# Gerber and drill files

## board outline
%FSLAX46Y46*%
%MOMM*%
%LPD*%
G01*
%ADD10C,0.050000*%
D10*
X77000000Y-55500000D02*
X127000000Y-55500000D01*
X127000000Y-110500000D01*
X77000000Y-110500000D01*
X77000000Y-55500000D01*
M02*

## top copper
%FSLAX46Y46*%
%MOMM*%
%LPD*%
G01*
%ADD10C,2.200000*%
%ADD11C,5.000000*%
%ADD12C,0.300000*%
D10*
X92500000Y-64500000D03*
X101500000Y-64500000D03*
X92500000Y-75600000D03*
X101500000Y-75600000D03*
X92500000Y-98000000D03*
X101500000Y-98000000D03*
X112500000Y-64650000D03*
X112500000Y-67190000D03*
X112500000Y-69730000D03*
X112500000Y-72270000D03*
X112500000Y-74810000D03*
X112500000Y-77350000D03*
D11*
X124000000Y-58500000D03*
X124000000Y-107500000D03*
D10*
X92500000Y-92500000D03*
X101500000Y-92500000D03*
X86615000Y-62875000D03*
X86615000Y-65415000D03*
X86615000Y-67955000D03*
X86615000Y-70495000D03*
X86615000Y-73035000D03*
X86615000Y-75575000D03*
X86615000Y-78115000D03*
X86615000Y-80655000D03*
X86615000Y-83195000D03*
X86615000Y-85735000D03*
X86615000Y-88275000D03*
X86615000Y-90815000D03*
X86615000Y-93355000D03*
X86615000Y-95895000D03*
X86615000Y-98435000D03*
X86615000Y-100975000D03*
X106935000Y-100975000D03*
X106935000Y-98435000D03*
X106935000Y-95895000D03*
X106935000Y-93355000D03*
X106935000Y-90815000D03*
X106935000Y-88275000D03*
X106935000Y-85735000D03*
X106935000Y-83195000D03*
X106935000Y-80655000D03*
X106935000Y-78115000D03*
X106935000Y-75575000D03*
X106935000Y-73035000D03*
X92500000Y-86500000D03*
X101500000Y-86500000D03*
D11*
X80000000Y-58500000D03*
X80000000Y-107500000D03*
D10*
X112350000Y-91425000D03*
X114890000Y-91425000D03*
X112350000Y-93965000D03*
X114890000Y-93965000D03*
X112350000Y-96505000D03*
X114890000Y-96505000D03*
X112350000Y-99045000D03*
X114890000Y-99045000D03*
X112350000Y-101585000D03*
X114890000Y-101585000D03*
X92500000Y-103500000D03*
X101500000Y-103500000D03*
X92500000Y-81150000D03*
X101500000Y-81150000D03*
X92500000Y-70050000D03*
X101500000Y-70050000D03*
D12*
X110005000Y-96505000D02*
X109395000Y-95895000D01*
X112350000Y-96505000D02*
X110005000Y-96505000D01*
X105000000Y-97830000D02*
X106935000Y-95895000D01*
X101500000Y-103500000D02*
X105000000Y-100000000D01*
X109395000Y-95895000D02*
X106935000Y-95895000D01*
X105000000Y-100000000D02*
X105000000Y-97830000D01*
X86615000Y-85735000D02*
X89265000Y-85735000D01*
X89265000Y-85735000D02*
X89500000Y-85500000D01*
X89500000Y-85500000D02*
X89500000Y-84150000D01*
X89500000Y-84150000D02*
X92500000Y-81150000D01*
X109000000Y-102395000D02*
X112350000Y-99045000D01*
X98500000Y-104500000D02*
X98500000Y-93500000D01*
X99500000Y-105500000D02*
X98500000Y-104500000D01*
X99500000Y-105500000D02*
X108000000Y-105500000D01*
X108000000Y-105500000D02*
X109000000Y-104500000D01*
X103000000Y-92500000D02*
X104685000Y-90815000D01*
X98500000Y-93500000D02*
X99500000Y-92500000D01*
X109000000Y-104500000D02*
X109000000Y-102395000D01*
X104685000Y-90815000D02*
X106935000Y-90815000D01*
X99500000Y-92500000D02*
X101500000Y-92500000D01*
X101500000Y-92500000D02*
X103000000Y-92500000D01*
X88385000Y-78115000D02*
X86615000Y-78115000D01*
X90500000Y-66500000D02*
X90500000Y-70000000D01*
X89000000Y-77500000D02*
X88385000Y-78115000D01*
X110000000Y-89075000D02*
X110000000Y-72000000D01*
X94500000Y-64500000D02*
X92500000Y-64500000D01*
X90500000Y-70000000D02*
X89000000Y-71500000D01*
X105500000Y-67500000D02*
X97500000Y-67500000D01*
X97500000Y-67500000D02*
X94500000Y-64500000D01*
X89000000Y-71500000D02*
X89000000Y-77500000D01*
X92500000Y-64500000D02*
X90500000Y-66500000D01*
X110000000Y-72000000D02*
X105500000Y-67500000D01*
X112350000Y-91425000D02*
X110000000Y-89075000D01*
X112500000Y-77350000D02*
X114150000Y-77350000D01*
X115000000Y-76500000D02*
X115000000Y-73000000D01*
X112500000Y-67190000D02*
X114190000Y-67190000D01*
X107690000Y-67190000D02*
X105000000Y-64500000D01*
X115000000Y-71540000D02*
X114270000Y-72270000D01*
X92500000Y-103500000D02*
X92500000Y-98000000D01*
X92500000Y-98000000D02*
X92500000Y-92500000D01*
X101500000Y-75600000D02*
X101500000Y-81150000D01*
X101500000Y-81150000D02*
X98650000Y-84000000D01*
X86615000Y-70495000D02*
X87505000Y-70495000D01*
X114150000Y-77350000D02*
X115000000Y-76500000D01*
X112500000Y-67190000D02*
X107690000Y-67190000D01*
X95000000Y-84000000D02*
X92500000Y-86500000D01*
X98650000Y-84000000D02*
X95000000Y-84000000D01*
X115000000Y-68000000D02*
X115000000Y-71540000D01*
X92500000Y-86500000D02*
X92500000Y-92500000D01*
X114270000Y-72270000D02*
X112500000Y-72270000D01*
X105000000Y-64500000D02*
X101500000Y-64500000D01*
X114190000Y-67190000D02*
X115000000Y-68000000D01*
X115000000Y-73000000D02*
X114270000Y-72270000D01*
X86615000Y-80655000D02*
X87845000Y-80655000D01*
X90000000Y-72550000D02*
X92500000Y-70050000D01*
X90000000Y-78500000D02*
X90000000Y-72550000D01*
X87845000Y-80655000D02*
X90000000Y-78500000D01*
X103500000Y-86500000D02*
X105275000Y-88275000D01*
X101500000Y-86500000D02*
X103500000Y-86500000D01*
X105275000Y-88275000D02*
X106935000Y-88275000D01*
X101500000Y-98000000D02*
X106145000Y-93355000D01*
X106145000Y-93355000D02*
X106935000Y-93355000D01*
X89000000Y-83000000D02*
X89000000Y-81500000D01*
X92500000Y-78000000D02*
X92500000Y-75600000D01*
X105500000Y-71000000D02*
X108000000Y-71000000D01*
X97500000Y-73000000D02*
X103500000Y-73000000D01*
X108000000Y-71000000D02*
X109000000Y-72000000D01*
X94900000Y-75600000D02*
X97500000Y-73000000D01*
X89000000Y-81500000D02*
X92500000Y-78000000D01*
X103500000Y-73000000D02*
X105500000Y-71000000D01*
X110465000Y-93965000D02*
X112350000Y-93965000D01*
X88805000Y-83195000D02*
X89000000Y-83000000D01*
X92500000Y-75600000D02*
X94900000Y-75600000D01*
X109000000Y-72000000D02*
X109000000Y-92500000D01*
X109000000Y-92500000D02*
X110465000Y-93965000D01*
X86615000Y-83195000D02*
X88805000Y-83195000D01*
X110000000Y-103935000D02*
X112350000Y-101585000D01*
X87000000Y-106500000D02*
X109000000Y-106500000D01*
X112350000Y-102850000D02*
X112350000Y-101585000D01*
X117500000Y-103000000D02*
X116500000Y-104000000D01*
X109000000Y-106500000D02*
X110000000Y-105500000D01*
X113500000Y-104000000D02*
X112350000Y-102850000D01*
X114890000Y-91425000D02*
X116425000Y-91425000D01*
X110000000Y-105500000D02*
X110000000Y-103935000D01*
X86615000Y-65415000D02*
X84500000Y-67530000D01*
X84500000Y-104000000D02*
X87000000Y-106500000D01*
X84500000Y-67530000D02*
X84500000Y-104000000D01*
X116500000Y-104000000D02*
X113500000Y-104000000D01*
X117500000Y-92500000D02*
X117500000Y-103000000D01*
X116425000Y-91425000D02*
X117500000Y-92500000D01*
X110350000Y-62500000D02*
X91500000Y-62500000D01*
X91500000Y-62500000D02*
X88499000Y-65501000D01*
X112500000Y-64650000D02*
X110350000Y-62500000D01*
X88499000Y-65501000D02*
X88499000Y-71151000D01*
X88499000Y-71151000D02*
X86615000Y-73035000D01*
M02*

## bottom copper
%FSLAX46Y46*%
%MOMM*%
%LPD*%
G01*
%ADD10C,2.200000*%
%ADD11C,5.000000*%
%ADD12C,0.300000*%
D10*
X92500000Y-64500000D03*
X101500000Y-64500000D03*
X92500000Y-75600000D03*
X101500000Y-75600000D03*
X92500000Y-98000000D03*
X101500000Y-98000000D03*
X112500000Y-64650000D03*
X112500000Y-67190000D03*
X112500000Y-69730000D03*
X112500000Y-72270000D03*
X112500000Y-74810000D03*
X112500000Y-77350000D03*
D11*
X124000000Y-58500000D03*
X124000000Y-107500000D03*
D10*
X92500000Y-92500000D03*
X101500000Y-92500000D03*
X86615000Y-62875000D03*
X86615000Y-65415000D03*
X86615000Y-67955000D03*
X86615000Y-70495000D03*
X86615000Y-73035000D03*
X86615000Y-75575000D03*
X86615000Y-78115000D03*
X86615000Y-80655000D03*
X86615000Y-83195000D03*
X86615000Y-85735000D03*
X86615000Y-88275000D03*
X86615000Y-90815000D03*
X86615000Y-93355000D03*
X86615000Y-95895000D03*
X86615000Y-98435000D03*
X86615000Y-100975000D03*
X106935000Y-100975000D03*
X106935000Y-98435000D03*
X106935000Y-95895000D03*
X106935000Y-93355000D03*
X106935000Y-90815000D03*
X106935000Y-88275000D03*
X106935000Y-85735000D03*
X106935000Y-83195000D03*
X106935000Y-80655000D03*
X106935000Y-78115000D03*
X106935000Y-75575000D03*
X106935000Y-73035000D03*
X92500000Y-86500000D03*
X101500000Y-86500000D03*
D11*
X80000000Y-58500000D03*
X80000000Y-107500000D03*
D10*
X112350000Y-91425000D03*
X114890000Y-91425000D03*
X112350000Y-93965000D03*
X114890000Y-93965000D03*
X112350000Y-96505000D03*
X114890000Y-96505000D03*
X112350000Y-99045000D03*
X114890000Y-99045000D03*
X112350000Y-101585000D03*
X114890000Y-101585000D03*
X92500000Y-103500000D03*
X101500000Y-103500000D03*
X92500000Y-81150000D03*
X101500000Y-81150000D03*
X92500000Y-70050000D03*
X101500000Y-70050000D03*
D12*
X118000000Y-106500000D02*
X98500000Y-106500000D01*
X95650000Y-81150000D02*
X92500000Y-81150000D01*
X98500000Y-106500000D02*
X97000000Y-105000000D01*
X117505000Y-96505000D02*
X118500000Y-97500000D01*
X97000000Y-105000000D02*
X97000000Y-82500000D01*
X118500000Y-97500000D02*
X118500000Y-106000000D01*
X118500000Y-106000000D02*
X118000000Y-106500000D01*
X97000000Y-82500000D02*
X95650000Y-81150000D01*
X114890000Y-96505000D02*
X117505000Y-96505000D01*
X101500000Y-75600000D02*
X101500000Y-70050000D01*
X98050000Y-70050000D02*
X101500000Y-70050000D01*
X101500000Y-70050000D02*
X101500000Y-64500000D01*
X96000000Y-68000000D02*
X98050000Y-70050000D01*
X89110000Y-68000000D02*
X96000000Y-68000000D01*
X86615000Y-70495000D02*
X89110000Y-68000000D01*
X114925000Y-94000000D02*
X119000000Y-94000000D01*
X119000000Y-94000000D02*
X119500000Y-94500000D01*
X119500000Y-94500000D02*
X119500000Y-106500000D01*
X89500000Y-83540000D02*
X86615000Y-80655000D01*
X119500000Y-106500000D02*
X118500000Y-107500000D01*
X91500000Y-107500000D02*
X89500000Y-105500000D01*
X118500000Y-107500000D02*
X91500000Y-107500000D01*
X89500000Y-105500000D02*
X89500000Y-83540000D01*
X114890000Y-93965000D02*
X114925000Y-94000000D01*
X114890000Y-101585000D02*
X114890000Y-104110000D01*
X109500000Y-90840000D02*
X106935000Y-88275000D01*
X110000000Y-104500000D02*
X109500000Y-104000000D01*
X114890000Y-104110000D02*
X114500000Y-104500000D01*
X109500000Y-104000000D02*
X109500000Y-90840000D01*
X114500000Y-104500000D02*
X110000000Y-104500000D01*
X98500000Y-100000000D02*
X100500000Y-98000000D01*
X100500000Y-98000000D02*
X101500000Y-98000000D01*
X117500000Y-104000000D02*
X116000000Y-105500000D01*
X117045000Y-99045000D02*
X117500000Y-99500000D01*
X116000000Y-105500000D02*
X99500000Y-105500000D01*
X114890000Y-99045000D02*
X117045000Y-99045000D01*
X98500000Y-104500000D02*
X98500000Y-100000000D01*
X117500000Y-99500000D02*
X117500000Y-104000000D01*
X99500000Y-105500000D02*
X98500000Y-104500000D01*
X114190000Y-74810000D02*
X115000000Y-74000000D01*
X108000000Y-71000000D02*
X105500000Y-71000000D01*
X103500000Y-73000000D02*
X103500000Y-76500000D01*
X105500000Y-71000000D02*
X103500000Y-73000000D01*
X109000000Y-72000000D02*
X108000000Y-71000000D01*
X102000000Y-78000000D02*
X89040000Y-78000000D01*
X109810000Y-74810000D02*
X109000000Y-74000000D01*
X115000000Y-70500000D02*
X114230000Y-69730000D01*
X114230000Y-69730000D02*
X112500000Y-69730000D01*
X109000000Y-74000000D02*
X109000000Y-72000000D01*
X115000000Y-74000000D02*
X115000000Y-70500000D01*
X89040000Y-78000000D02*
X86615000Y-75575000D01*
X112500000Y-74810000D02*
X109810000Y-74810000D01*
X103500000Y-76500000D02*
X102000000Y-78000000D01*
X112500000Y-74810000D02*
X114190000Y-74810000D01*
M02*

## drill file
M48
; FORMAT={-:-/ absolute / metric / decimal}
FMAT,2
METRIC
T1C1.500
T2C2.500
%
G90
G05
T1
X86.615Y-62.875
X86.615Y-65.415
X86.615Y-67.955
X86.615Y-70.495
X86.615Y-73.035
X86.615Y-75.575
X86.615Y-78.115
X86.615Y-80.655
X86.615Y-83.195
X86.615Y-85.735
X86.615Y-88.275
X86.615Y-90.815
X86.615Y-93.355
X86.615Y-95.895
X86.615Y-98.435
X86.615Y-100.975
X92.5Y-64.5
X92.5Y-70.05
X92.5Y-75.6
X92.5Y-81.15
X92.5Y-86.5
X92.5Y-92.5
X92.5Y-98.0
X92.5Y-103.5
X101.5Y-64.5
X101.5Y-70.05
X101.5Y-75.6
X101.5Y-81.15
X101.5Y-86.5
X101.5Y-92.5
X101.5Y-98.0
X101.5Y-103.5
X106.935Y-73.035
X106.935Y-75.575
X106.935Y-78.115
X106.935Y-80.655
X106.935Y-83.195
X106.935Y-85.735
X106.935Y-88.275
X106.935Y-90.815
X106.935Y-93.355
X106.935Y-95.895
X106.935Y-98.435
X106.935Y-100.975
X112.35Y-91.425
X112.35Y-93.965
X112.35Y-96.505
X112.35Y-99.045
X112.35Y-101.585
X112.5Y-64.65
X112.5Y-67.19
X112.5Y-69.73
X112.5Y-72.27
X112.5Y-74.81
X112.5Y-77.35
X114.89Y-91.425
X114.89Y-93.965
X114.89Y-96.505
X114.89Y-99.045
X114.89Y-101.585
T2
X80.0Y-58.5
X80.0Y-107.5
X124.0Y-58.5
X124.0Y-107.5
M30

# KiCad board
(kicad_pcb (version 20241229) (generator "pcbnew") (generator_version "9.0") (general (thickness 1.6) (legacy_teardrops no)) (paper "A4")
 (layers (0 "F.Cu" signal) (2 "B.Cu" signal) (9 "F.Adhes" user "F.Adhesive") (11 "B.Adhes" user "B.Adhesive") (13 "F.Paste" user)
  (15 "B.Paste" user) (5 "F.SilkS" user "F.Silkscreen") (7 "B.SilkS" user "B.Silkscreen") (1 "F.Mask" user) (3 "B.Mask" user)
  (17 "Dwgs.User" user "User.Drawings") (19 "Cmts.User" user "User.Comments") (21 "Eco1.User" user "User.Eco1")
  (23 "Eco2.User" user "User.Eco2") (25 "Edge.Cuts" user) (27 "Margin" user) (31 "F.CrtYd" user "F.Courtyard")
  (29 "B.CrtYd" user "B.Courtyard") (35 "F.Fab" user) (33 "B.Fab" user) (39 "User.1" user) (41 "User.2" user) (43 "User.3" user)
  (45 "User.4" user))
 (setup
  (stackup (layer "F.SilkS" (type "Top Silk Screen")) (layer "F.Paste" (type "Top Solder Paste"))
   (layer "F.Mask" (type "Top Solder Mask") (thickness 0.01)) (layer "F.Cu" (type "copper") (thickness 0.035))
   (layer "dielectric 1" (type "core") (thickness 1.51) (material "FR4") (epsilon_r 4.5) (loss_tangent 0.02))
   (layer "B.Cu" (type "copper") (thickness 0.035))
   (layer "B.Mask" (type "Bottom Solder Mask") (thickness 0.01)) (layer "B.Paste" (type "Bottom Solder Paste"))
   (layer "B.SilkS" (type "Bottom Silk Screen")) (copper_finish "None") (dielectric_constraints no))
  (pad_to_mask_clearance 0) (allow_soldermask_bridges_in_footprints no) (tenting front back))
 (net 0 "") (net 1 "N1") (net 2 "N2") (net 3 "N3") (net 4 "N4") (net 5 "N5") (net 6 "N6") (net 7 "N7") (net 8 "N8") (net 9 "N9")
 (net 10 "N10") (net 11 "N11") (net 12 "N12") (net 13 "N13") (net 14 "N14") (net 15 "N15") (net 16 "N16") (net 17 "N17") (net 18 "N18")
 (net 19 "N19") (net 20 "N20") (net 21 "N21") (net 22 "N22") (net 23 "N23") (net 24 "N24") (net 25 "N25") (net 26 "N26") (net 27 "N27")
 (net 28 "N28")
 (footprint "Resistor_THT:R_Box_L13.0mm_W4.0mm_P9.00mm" (layer "F.Cu") (at 92.5 64.5)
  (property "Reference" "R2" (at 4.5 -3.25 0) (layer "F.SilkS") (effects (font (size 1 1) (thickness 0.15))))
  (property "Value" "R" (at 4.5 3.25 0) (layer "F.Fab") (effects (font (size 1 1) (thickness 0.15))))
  (pad "1" thru_hole circle (at 0 0) (size 2.2 2.2) (drill 1.5) (layers "*.Cu" "*.Mask") (remove_unused_layers no) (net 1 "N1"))
  (pad "2" thru_hole circle (at 9 0) (size 2.2 2.2) (drill 1.5) (layers "*.Cu" "*.Mask") (remove_unused_layers no) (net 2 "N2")))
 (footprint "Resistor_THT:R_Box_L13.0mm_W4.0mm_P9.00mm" (layer "F.Cu") (at 92.5 75.6)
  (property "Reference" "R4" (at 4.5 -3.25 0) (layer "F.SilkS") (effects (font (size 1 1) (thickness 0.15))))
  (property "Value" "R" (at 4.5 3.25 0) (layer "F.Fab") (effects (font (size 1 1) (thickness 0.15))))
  (pad "1" thru_hole circle (at 0 0) (size 2.2 2.2) (drill 1.5) (layers "*.Cu" "*.Mask") (remove_unused_layers no) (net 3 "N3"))
  (pad "2" thru_hole circle (at 9 0) (size 2.2 2.2) (drill 1.5) (layers "*.Cu" "*.Mask") (remove_unused_layers no) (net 2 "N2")))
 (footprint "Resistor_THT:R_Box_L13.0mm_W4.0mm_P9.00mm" (layer "F.Cu") (at 92.5 98)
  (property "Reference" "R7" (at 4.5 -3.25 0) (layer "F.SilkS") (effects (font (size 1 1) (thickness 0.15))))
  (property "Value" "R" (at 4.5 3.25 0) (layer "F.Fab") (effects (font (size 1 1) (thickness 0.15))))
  (pad "1" thru_hole circle (at 0 0) (size 2.2 2.2) (drill 1.5) (layers "*.Cu" "*.Mask") (remove_unused_layers no) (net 2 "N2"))
  (pad "2" thru_hole circle (at 9 0) (size 2.2 2.2) (drill 1.5) (layers "*.Cu" "*.Mask") (remove_unused_layers no) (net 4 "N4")))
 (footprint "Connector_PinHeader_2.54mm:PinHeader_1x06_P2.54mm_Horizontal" (layer "F.Cu") (at 112.5 64.65)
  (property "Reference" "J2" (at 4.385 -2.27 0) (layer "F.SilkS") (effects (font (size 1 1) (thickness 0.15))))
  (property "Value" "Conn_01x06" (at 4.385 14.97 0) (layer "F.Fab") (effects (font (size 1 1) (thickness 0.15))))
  (pad "1" thru_hole circle (at 0 0) (size 2.2 2.2) (drill 1.5) (layers "*.Cu" "*.Mask") (remove_unused_layers no) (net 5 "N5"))
  (pad "2" thru_hole circle (at 0 2.54) (size 2.2 2.2) (drill 1.5) (layers "*.Cu" "*.Mask") (remove_unused_layers no) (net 2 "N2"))
  (pad "3" thru_hole circle (at 0 5.08) (size 2.2 2.2) (drill 1.5) (layers "*.Cu" "*.Mask") (remove_unused_layers no) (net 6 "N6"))
  (pad "4" thru_hole circle (at 0 7.62) (size 2.2 2.2) (drill 1.5) (layers "*.Cu" "*.Mask") (remove_unused_layers no) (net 2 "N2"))
  (pad "5" thru_hole circle (at 0 10.16) (size 2.2 2.2) (drill 1.5) (layers "*.Cu" "*.Mask") (remove_unused_layers no) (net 6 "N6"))
  (pad "6" thru_hole circle (at 0 12.7) (size 2.2 2.2) (drill 1.5) (layers "*.Cu" "*.Mask") (remove_unused_layers no) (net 2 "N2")))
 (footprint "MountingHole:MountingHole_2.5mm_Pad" (layer "F.Cu") (at 124 58.5)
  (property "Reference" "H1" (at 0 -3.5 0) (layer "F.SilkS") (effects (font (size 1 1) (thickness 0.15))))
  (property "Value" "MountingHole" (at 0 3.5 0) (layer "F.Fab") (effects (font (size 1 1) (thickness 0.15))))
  (pad "1" thru_hole circle (at 0 0) (size 5 5) (drill 2.5) (layers "*.Cu" "*.Mask") (remove_unused_layers no)))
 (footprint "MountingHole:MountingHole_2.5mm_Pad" (layer "F.Cu") (at 124 107.5)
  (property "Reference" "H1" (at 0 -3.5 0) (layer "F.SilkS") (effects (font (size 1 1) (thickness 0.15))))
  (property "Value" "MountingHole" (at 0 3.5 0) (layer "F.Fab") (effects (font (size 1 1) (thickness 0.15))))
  (pad "1" thru_hole circle (at 0 0) (size 5 5) (drill 2.5) (layers "*.Cu" "*.Mask") (remove_unused_layers no)))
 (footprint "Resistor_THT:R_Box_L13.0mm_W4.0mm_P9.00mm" (layer "F.Cu") (at 92.5 92.5)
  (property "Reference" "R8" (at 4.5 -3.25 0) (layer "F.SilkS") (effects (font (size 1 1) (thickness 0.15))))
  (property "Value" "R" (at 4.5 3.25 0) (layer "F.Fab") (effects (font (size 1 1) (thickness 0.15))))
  (pad "1" thru_hole circle (at 0 0) (size 2.2 2.2) (drill 1.5) (layers "*.Cu" "*.Mask") (remove_unused_layers no) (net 2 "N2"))
  (pad "2" thru_hole circle (at 9 0) (size 2.2 2.2) (drill 1.5) (layers "*.Cu" "*.Mask") (remove_unused_layers no) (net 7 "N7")))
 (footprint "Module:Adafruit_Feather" (layer "F.Cu") (at 86.615 62.875)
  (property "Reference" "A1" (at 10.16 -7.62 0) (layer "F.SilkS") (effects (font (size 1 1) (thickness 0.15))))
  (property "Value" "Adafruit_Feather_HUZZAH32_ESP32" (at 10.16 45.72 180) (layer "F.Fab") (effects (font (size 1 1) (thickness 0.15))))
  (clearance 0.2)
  (pad "1" thru_hole circle (at 0 0) (size 2.2 2.2) (drill 1.5) (layers "*.Cu" "*.Mask") (remove_unused_layers no) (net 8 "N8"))
  (pad "2" thru_hole circle (at 0 2.54) (size 2.2 2.2) (drill 1.5) (layers "*.Cu" "*.Mask") (remove_unused_layers no) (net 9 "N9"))
  (pad "3" thru_hole circle (at 0 5.08) (size 2.2 2.2) (drill 1.5) (layers "*.Cu" "*.Mask") (remove_unused_layers no) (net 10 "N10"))
  (pad "4" thru_hole circle (at 0 7.62) (size 2.2 2.2) (drill 1.5) (layers "*.Cu" "*.Mask") (remove_unused_layers no) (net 2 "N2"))
  (pad "5" thru_hole circle (at 0 10.16) (size 2.2 2.2) (drill 1.5) (layers "*.Cu" "*.Mask") (remove_unused_layers no) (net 5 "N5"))
  (pad "6" thru_hole circle (at 0 12.7) (size 2.2 2.2) (drill 1.5) (layers "*.Cu" "*.Mask") (remove_unused_layers no) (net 6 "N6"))
  (pad "7" thru_hole circle (at 0 15.24) (size 2.2 2.2) (drill 1.5) (layers "*.Cu" "*.Mask") (remove_unused_layers no) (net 1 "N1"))
  (pad "8" thru_hole circle (at 0 17.78) (size 2.2 2.2) (drill 1.5) (layers "*.Cu" "*.Mask") (remove_unused_layers no) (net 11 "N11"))
  (pad "9" thru_hole circle (at 0 20.32) (size 2.2 2.2) (drill 1.5) (layers "*.Cu" "*.Mask") (remove_unused_layers no) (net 3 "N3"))
  (pad "10" thru_hole circle (at 0 22.86) (size 2.2 2.2) (drill 1.5) (layers "*.Cu" "*.Mask") (remove_unused_layers no) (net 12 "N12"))
  (pad "11" thru_hole circle (at 0 25.4) (size 2.2 2.2) (drill 1.5) (layers "*.Cu" "*.Mask") (remove_unused_layers no) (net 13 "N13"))
  (pad "12" thru_hole circle (at 0 27.94) (size 2.2 2.2) (drill 1.5) (layers "*.Cu" "*.Mask") (remove_unused_layers no) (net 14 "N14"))
  (pad "13" thru_hole circle (at 0 30.48) (size 2.2 2.2) (drill 1.5) (layers "*.Cu" "*.Mask") (remove_unused_layers no) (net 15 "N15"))
  (pad "14" thru_hole circle (at 0 33.02) (size 2.2 2.2) (drill 1.5) (layers "*.Cu" "*.Mask") (remove_unused_layers no) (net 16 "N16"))
  (pad "15" thru_hole circle (at 0 35.56) (size 2.2 2.2) (drill 1.5) (layers "*.Cu" "*.Mask") (remove_unused_layers no) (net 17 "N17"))
  (pad "16" thru_hole circle (at 0 38.1) (size 2.2 2.2) (drill 1.5) (layers "*.Cu" "*.Mask") (remove_unused_layers no) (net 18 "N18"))
  (pad "17" thru_hole circle (at 20.32 38.1) (size 2.2 2.2) (drill 1.5) (layers "*.Cu" "*.Mask") (remove_unused_layers no) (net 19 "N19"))
  (pad "18" thru_hole circle (at 20.32 35.56) (size 2.2 2.2) (drill 1.5) (layers "*.Cu" "*.Mask") (remove_unused_layers no) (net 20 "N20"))
  (pad "19" thru_hole circle (at 20.32 33.02) (size 2.2 2.2) (drill 1.5) (layers "*.Cu" "*.Mask") (remove_unused_layers no) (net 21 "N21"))
  (pad "20" thru_hole circle (at 20.32 30.48) (size 2.2 2.2) (drill 1.5) (layers "*.Cu" "*.Mask") (remove_unused_layers no) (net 4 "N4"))
  (pad "21" thru_hole circle (at 20.32 27.94) (size 2.2 2.2) (drill 1.5) (layers "*.Cu" "*.Mask") (remove_unused_layers no) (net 7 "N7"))
  (pad "22" thru_hole circle (at 20.32 25.4) (size 2.2 2.2) (drill 1.5) (layers "*.Cu" "*.Mask") (remove_unused_layers no) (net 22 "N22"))
  (pad "23" thru_hole circle (at 20.32 22.86) (size 2.2 2.2) (drill 1.5) (layers "*.Cu" "*.Mask") (remove_unused_layers no) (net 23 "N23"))
  (pad "24" thru_hole circle (at 20.32 20.32) (size 2.2 2.2) (drill 1.5) (layers "*.Cu" "*.Mask") (remove_unused_layers no) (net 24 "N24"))
  (pad "25" thru_hole circle (at 20.32 17.78) (size 2.2 2.2) (drill 1.5) (layers "*.Cu" "*.Mask") (remove_unused_layers no) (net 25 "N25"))
  (pad "26" thru_hole circle (at 20.32 15.24) (size 2.2 2.2) (drill 1.5) (layers "*.Cu" "*.Mask") (remove_unused_layers no) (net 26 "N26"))
  (pad "27" thru_hole circle (at 20.32 12.7) (size 2.2 2.2) (drill 1.5) (layers "*.Cu" "*.Mask") (remove_unused_layers no) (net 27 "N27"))
  (pad "28" thru_hole circle (at 20.32 10.16) (size 2.2 2.2) (drill 1.5) (layers "*.Cu" "*.Mask") (remove_unused_layers no) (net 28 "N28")))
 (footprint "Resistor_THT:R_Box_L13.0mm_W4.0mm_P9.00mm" (layer "F.Cu") (at 92.5 86.5)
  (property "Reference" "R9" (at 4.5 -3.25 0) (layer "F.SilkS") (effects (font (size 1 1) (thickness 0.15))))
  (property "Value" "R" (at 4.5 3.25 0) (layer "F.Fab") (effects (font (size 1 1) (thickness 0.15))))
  (pad "1" thru_hole circle (at 0 0) (size 2.2 2.2) (drill 1.5) (layers "*.Cu" "*.Mask") (remove_unused_layers no) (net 2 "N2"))
  (pad "2" thru_hole circle (at 9 0) (size 2.2 2.2) (drill 1.5) (layers "*.Cu" "*.Mask") (remove_unused_layers no) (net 22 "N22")))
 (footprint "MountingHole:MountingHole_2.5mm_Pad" (layer "F.Cu") (at 80 58.5)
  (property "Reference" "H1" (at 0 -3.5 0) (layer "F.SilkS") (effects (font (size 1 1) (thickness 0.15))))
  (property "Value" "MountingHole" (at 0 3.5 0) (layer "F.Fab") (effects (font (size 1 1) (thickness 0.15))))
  (pad "1" thru_hole circle (at 0 0) (size 5 5) (drill 2.5) (layers "*.Cu" "*.Mask") (remove_unused_layers no)))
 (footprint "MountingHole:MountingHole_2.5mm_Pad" (layer "F.Cu") (at 80 107.5)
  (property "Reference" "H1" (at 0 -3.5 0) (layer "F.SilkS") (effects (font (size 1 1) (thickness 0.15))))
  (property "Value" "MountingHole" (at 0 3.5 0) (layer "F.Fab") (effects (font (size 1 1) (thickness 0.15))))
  (pad "1" thru_hole circle (at 0 0) (size 5 5) (drill 2.5) (layers "*.Cu" "*.Mask") (remove_unused_layers no)))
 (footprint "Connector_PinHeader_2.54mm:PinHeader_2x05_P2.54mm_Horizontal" (layer "F.Cu") (at 112.35 91.425)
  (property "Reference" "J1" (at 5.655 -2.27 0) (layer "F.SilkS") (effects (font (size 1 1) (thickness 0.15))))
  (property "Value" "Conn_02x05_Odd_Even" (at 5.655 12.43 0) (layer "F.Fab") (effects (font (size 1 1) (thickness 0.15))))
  (pad "1" thru_hole circle (at 0 0) (size 2.2 2.2) (drill 1.5) (layers "*.Cu" "*.Mask") (remove_unused_layers no) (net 1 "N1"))
  (pad "2" thru_hole circle (at 2.54 0) (size 2.2 2.2) (drill 1.5) (layers "*.Cu" "*.Mask") (remove_unused_layers no) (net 9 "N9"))
  (pad "3" thru_hole circle (at 0 2.54) (size 2.2 2.2) (drill 1.5) (layers "*.Cu" "*.Mask") (remove_unused_layers no) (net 3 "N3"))
  (pad "4" thru_hole circle (at 2.54 2.54) (size 2.2 2.2) (drill 1.5) (layers "*.Cu" "*.Mask") (remove_unused_layers no) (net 11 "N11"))
  (pad "5" thru_hole circle (at 0 5.08) (size 2.2 2.2) (drill 1.5) (layers "*.Cu" "*.Mask") (remove_unused_layers no) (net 21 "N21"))
  (pad "6" thru_hole circle (at 2.54 5.08) (size 2.2 2.2) (drill 1.5) (layers "*.Cu" "*.Mask") (remove_unused_layers no) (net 12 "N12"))
  (pad "7" thru_hole circle (at 0 7.62) (size 2.2 2.2) (drill 1.5) (layers "*.Cu" "*.Mask") (remove_unused_layers no) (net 7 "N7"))
  (pad "8" thru_hole circle (at 2.54 7.62) (size 2.2 2.2) (drill 1.5) (layers "*.Cu" "*.Mask") (remove_unused_layers no) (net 4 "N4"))
  (pad "9" thru_hole circle (at 0 10.16) (size 2.2 2.2) (drill 1.5) (layers "*.Cu" "*.Mask") (remove_unused_layers no) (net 9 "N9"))
  (pad "10" thru_hole circle (at 2.54 10.16) (size 2.2 2.2) (drill 1.5) (layers "*.Cu" "*.Mask") (remove_unused_layers no) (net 22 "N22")))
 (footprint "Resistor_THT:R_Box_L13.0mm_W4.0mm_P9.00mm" (layer "F.Cu") (at 92.5 103.5)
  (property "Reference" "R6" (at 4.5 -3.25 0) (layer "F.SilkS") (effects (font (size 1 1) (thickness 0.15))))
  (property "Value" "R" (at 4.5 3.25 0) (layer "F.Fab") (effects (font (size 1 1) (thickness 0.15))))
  (pad "1" thru_hole circle (at 0 0) (size 2.2 2.2) (drill 1.5) (layers "*.Cu" "*.Mask") (remove_unused_layers no) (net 2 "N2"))
  (pad "2" thru_hole circle (at 9 0) (size 2.2 2.2) (drill 1.5) (layers "*.Cu" "*.Mask") (remove_unused_layers no) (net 21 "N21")))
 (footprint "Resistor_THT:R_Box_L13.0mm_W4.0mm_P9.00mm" (layer "F.Cu") (at 92.5 81.15)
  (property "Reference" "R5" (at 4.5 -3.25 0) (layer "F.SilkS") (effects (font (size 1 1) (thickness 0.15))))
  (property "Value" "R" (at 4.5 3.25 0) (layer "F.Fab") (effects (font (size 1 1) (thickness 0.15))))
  (pad "1" thru_hole circle (at 0 0) (size 2.2 2.2) (drill 1.5) (layers "*.Cu" "*.Mask") (remove_unused_layers no) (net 12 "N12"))
  (pad "2" thru_hole circle (at 9 0) (size 2.2 2.2) (drill 1.5) (layers "*.Cu" "*.Mask") (remove_unused_layers no) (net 2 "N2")))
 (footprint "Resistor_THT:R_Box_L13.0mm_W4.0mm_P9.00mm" (layer "F.Cu") (at 92.5 70.05)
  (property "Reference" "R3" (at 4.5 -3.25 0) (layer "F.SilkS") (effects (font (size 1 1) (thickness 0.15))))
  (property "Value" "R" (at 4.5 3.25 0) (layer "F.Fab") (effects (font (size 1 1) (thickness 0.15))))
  (pad "1" thru_hole circle (at 0 0) (size 2.2 2.2) (drill 1.5) (layers "*.Cu" "*.Mask") (remove_unused_layers no) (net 11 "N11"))
  (pad "2" thru_hole circle (at 9 0) (size 2.2 2.2) (drill 1.5) (layers "*.Cu" "*.Mask") (remove_unused_layers no) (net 2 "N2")))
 (gr_rect (start 77 55.5) (end 127 110.5) (stroke (width 0.05) (type default)) (fill no) (layer "Edge.Cuts"))
 (segment (start 110.005 96.505) (end 109.395 95.895) (width 0.3) (layer "F.Cu") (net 21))
 (segment (start 112.35 96.505) (end 110.005 96.505) (width 0.3) (layer "F.Cu") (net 21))
 (segment (start 105 97.83) (end 106.935 95.895) (width 0.3) (layer "F.Cu") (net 21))
 (segment (start 101.5 103.5) (end 105 100) (width 0.3) (layer "F.Cu") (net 21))
 (segment (start 109.395 95.895) (end 106.935 95.895) (width 0.3) (layer "F.Cu") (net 21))
 (segment (start 105 100) (end 105 97.83) (width 0.3) (layer "F.Cu") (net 21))
 (segment (start 86.615 85.735) (end 89.265 85.735) (width 0.3) (layer "F.Cu") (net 12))
 (segment (start 89.265 85.735) (end 89.5 85.5) (width 0.3) (layer "F.Cu") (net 12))
 (segment (start 89.5 85.5) (end 89.5 84.15) (width 0.3) (layer "F.Cu") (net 12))
 (segment (start 89.5 84.15) (end 92.5 81.15) (width 0.3) (layer "F.Cu") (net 12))
 (segment (start 118 106.5) (end 98.5 106.5) (width 0.3) (layer "B.Cu") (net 12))
 (segment (start 95.65 81.15) (end 92.5 81.15) (width 0.3) (layer "B.Cu") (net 12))
 (segment (start 98.5 106.5) (end 97 105) (width 0.3) (layer "B.Cu") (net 12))
 (segment (start 117.505 96.505) (end 118.5 97.5) (width 0.3) (layer "B.Cu") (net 12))
 (segment (start 97 105) (end 97 82.5) (width 0.3) (layer "B.Cu") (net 12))
 (segment (start 118.5 97.5) (end 118.5 106) (width 0.3) (layer "B.Cu") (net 12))
 (segment (start 118.5 106) (end 118 106.5) (width 0.3) (layer "B.Cu") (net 12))
 (segment (start 97 82.5) (end 95.65 81.15) (width 0.3) (layer "B.Cu") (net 12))
 (segment (start 114.89 96.505) (end 117.505 96.505) (width 0.3) (layer "B.Cu") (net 12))
 (segment (start 109 102.395) (end 112.35 99.045) (width 0.3) (layer "F.Cu") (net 7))
 (segment (start 98.5 104.5) (end 98.5 93.5) (width 0.3) (layer "F.Cu") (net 7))
 (segment (start 99.5 105.5) (end 98.5 104.5) (width 0.3) (layer "F.Cu") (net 7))
 (segment (start 99.5 105.5) (end 108 105.5) (width 0.3) (layer "F.Cu") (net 7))
 (segment (start 108 105.5) (end 109 104.5) (width 0.3) (layer "F.Cu") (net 7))
 (segment (start 103 92.5) (end 104.685 90.815) (width 0.3) (layer "F.Cu") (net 7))
 (segment (start 98.5 93.5) (end 99.5 92.5) (width 0.3) (layer "F.Cu") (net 7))
 (segment (start 109 104.5) (end 109 102.395) (width 0.3) (layer "F.Cu") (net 7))
 (segment (start 104.685 90.815) (end 106.935 90.815) (width 0.3) (layer "F.Cu") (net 7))
 (segment (start 99.5 92.5) (end 101.5 92.5) (width 0.3) (layer "F.Cu") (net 7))
 (segment (start 101.5 92.5) (end 103 92.5) (width 0.3) (layer "F.Cu") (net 7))
 (segment (start 88.385 78.115) (end 86.615 78.115) (width 0.3) (layer "F.Cu") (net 1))
 (segment (start 90.5 66.5) (end 90.5 70) (width 0.3) (layer "F.Cu") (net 1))
 (segment (start 89 77.5) (end 88.385 78.115) (width 0.3) (layer "F.Cu") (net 1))
 (segment (start 110 89.075) (end 110 72) (width 0.3) (layer "F.Cu") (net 1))
 (segment (start 94.5 64.5) (end 92.5 64.5) (width 0.3) (layer "F.Cu") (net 1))
 (segment (start 90.5 70) (end 89 71.5) (width 0.3) (layer "F.Cu") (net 1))
 (segment (start 105.5 67.5) (end 97.5 67.5) (width 0.3) (layer "F.Cu") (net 1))
 (segment (start 97.5 67.5) (end 94.5 64.5) (width 0.3) (layer "F.Cu") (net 1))
 (segment (start 89 71.5) (end 89 77.5) (width 0.3) (layer "F.Cu") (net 1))
 (segment (start 92.5 64.5) (end 90.5 66.5) (width 0.3) (layer "F.Cu") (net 1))
 (segment (start 110 72) (end 105.5 67.5) (width 0.3) (layer "F.Cu") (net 1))
 (segment (start 112.35 91.425) (end 110 89.075) (width 0.3) (layer "F.Cu") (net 1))
 (segment (start 112.5 77.35) (end 114.15 77.35) (width 0.3) (layer "F.Cu") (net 2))
 (segment (start 115 76.5) (end 115 73) (width 0.3) (layer "F.Cu") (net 2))
 (segment (start 112.5 67.19) (end 114.19 67.19) (width 0.3) (layer "F.Cu") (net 2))
 (segment (start 107.69 67.19) (end 105 64.5) (width 0.3) (layer "F.Cu") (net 2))
 (segment (start 115 71.54) (end 114.27 72.27) (width 0.3) (layer "F.Cu") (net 2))
 (segment (start 92.5 103.5) (end 92.5 98) (width 0.3) (layer "F.Cu") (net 2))
 (segment (start 92.5 98) (end 92.5 92.5) (width 0.3) (layer "F.Cu") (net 2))
 (segment (start 101.5 75.6) (end 101.5 81.15) (width 0.3) (layer "F.Cu") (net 2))
 (segment (start 101.5 81.15) (end 98.65 84) (width 0.3) (layer "F.Cu") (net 2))
 (segment (start 86.615 70.495) (end 87.505 70.495) (width 0.3) (layer "F.Cu") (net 2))
 (segment (start 114.15 77.35) (end 115 76.5) (width 0.3) (layer "F.Cu") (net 2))
 (segment (start 112.5 67.19) (end 107.69 67.19) (width 0.3) (layer "F.Cu") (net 2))
 (segment (start 95 84) (end 92.5 86.5) (width 0.3) (layer "F.Cu") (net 2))
 (segment (start 98.65 84) (end 95 84) (width 0.3) (layer "F.Cu") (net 2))
 (segment (start 115 68) (end 115 71.54) (width 0.3) (layer "F.Cu") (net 2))
 (segment (start 92.5 86.5) (end 92.5 92.5) (width 0.3) (layer "F.Cu") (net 2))
 (segment (start 114.27 72.27) (end 112.5 72.27) (width 0.3) (layer "F.Cu") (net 2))
 (segment (start 105 64.5) (end 101.5 64.5) (width 0.3) (layer "F.Cu") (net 2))
 (segment (start 114.19 67.19) (end 115 68) (width 0.3) (layer "F.Cu") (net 2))
 (segment (start 115 73) (end 114.27 72.27) (width 0.3) (layer "F.Cu") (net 2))
 (segment (start 101.5 75.6) (end 101.5 70.05) (width 0.3) (layer "B.Cu") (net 2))
 (segment (start 98.05 70.05) (end 101.5 70.05) (width 0.3) (layer "B.Cu") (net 2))
 (segment (start 101.5 70.05) (end 101.5 64.5) (width 0.3) (layer "B.Cu") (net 2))
 (segment (start 96 68) (end 98.05 70.05) (width 0.3) (layer "B.Cu") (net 2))
 (segment (start 89.11 68) (end 96 68) (width 0.3) (layer "B.Cu") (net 2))
 (segment (start 86.615 70.495) (end 89.11 68) (width 0.3) (layer "B.Cu") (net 2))
 (segment (start 86.615 80.655) (end 87.845 80.655) (width 0.3) (layer "F.Cu") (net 11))
 (segment (start 90 72.55) (end 92.5 70.05) (width 0.3) (layer "F.Cu") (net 11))
 (segment (start 90 78.5) (end 90 72.55) (width 0.3) (layer "F.Cu") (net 11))
 (segment (start 87.845 80.655) (end 90 78.5) (width 0.3) (layer "F.Cu") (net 11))
 (segment (start 114.925 94) (end 119 94) (width 0.3) (layer "B.Cu") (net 11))
 (segment (start 119 94) (end 119.5 94.5) (width 0.3) (layer "B.Cu") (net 11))
 (segment (start 119.5 94.5) (end 119.5 106.5) (width 0.3) (layer "B.Cu") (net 11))
 (segment (start 89.5 83.54) (end 86.615 80.655) (width 0.3) (layer "B.Cu") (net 11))
 (segment (start 119.5 106.5) (end 118.5 107.5) (width 0.3) (layer "B.Cu") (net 11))
 (segment (start 91.5 107.5) (end 89.5 105.5) (width 0.3) (layer "B.Cu") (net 11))
 (segment (start 118.5 107.5) (end 91.5 107.5) (width 0.3) (layer "B.Cu") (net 11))
 (segment (start 89.5 105.5) (end 89.5 83.54) (width 0.3) (layer "B.Cu") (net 11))
 (segment (start 114.89 93.965) (end 114.925 94) (width 0.3) (layer "B.Cu") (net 11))
 (segment (start 103.5 86.5) (end 105.275 88.275) (width 0.3) (layer "F.Cu") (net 22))
 (segment (start 101.5 86.5) (end 103.5 86.5) (width 0.3) (layer "F.Cu") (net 22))
 (segment (start 105.275 88.275) (end 106.935 88.275) (width 0.3) (layer "F.Cu") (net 22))
 (segment (start 114.89 101.585) (end 114.89 104.11) (width 0.3) (layer "B.Cu") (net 22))
 (segment (start 109.5 90.84) (end 106.935 88.275) (width 0.3) (layer "B.Cu") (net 22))
 (segment (start 110 104.5) (end 109.5 104) (width 0.3) (layer "B.Cu") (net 22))
 (segment (start 114.89 104.11) (end 114.5 104.5) (width 0.3) (layer "B.Cu") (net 22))
 (segment (start 109.5 104) (end 109.5 90.84) (width 0.3) (layer "B.Cu") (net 22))
 (segment (start 114.5 104.5) (end 110 104.5) (width 0.3) (layer "B.Cu") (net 22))
 (segment (start 101.5 98) (end 106.145 93.355) (width 0.3) (layer "F.Cu") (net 4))
 (segment (start 106.145 93.355) (end 106.935 93.355) (width 0.3) (layer "F.Cu") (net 4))
 (segment (start 98.5 100) (end 100.5 98) (width 0.3) (layer "B.Cu") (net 4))
 (segment (start 100.5 98) (end 101.5 98) (width 0.3) (layer "B.Cu") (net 4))
 (segment (start 117.5 104) (end 116 105.5) (width 0.3) (layer "B.Cu") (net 4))
 (segment (start 117.045 99.045) (end 117.5 99.5) (width 0.3) (layer "B.Cu") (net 4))
 (segment (start 116 105.5) (end 99.5 105.5) (width 0.3) (layer "B.Cu") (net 4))
 (segment (start 114.89 99.045) (end 117.045 99.045) (width 0.3) (layer "B.Cu") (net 4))
 (segment (start 98.5 104.5) (end 98.5 100) (width 0.3) (layer "B.Cu") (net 4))
 (segment (start 117.5 99.5) (end 117.5 104) (width 0.3) (layer "B.Cu") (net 4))
 (segment (start 99.5 105.5) (end 98.5 104.5) (width 0.3) (layer "B.Cu") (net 4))
 (segment (start 89 83) (end 89 81.5) (width 0.3) (layer "F.Cu") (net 3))
 (segment (start 92.5 78) (end 92.5 75.6) (width 0.3) (layer "F.Cu") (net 3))
 (segment (start 105.5 71) (end 108 71) (width 0.3) (layer "F.Cu") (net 3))
 (segment (start 97.5 73) (end 103.5 73) (width 0.3) (layer "F.Cu") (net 3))
 (segment (start 108 71) (end 109 72) (width 0.3) (layer "F.Cu") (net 3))
 (segment (start 94.9 75.6) (end 97.5 73) (width 0.3) (layer "F.Cu") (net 3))
 (segment (start 89 81.5) (end 92.5 78) (width 0.3) (layer "F.Cu") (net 3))
 (segment (start 103.5 73) (end 105.5 71) (width 0.3) (layer "F.Cu") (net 3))
 (segment (start 110.465 93.965) (end 112.35 93.965) (width 0.3) (layer "F.Cu") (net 3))
 (segment (start 88.805 83.195) (end 89 83) (width 0.3) (layer "F.Cu") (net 3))
 (segment (start 92.5 75.6) (end 94.9 75.6) (width 0.3) (layer "F.Cu") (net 3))
 (segment (start 109 72) (end 109 92.5) (width 0.3) (layer "F.Cu") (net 3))
 (segment (start 109 92.5) (end 110.465 93.965) (width 0.3) (layer "F.Cu") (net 3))
 (segment (start 86.615 83.195) (end 88.805 83.195) (width 0.3) (layer "F.Cu") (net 3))
 (segment (start 110 103.935) (end 112.35 101.585) (width 0.3) (layer "F.Cu") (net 9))
 (segment (start 87 106.5) (end 109 106.5) (width 0.3) (layer "F.Cu") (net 9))
 (segment (start 112.35 102.85) (end 112.35 101.585) (width 0.3) (layer "F.Cu") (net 9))
 (segment (start 117.5 103) (end 116.5 104) (width 0.3) (layer "F.Cu") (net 9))
 (segment (start 109 106.5) (end 110 105.5) (width 0.3) (layer "F.Cu") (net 9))
 (segment (start 113.5 104) (end 112.35 102.85) (width 0.3) (layer "F.Cu") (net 9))
 (segment (start 114.89 91.425) (end 116.425 91.425) (width 0.3) (layer "F.Cu") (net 9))
 (segment (start 110 105.5) (end 110 103.935) (width 0.3) (layer "F.Cu") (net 9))
 (segment (start 86.615 65.415) (end 84.5 67.53) (width 0.3) (layer "F.Cu") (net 9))
 (segment (start 84.5 104) (end 87 106.5) (width 0.3) (layer "F.Cu") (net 9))
 (segment (start 84.5 67.53) (end 84.5 104) (width 0.3) (layer "F.Cu") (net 9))
 (segment (start 116.5 104) (end 113.5 104) (width 0.3) (layer "F.Cu") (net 9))
 (segment (start 117.5 92.5) (end 117.5 103) (width 0.3) (layer "F.Cu") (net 9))
 (segment (start 116.425 91.425) (end 117.5 92.5) (width 0.3) (layer "F.Cu") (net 9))
 (segment (start 110.35 62.5) (end 91.5 62.5) (width 0.3) (layer "F.Cu") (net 5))
 (segment (start 91.5 62.5) (end 88.499 65.501) (width 0.3) (layer "F.Cu") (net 5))
 (segment (start 112.5 64.65) (end 110.35 62.5) (width 0.3) (layer "F.Cu") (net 5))
 (segment (start 88.499 65.501) (end 88.499 71.151) (width 0.3) (layer "F.Cu") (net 5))
 (segment (start 88.499 71.151) (end 86.615 73.035) (width 0.3) (layer "F.Cu") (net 5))
 (segment (start 114.19 74.81) (end 115 74) (width 0.3) (layer "B.Cu") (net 6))
 (segment (start 108 71) (end 105.5 71) (width 0.3) (layer "B.Cu") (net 6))
 (segment (start 103.5 73) (end 103.5 76.5) (width 0.3) (layer "B.Cu") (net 6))
 (segment (start 105.5 71) (end 103.5 73) (width 0.3) (layer "B.Cu") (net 6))
 (segment (start 109 72) (end 108 71) (width 0.3) (layer "B.Cu") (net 6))
 (segment (start 102 78) (end 89.04 78) (width 0.3) (layer "B.Cu") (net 6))
 (segment (start 109.81 74.81) (end 109 74) (width 0.3) (layer "B.Cu") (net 6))
 (segment (start 115 70.5) (end 114.23 69.73) (width 0.3) (layer "B.Cu") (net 6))
 (segment (start 114.23 69.73) (end 112.5 69.73) (width 0.3) (layer "B.Cu") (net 6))
 (segment (start 109 74) (end 109 72) (width 0.3) (layer "B.Cu") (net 6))
 (segment (start 115 74) (end 115 70.5) (width 0.3) (layer "B.Cu") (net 6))
 (segment (start 89.04 78) (end 86.615 75.575) (width 0.3) (layer "B.Cu") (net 6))
 (segment (start 112.5 74.81) (end 109.81 74.81) (width 0.3) (layer "B.Cu") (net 6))
 (segment (start 103.5 76.5) (end 102 78) (width 0.3) (layer "B.Cu") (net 6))
 (segment (start 112.5 74.81) (end 114.19 74.81) (width 0.3) (layer "B.Cu") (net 6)))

